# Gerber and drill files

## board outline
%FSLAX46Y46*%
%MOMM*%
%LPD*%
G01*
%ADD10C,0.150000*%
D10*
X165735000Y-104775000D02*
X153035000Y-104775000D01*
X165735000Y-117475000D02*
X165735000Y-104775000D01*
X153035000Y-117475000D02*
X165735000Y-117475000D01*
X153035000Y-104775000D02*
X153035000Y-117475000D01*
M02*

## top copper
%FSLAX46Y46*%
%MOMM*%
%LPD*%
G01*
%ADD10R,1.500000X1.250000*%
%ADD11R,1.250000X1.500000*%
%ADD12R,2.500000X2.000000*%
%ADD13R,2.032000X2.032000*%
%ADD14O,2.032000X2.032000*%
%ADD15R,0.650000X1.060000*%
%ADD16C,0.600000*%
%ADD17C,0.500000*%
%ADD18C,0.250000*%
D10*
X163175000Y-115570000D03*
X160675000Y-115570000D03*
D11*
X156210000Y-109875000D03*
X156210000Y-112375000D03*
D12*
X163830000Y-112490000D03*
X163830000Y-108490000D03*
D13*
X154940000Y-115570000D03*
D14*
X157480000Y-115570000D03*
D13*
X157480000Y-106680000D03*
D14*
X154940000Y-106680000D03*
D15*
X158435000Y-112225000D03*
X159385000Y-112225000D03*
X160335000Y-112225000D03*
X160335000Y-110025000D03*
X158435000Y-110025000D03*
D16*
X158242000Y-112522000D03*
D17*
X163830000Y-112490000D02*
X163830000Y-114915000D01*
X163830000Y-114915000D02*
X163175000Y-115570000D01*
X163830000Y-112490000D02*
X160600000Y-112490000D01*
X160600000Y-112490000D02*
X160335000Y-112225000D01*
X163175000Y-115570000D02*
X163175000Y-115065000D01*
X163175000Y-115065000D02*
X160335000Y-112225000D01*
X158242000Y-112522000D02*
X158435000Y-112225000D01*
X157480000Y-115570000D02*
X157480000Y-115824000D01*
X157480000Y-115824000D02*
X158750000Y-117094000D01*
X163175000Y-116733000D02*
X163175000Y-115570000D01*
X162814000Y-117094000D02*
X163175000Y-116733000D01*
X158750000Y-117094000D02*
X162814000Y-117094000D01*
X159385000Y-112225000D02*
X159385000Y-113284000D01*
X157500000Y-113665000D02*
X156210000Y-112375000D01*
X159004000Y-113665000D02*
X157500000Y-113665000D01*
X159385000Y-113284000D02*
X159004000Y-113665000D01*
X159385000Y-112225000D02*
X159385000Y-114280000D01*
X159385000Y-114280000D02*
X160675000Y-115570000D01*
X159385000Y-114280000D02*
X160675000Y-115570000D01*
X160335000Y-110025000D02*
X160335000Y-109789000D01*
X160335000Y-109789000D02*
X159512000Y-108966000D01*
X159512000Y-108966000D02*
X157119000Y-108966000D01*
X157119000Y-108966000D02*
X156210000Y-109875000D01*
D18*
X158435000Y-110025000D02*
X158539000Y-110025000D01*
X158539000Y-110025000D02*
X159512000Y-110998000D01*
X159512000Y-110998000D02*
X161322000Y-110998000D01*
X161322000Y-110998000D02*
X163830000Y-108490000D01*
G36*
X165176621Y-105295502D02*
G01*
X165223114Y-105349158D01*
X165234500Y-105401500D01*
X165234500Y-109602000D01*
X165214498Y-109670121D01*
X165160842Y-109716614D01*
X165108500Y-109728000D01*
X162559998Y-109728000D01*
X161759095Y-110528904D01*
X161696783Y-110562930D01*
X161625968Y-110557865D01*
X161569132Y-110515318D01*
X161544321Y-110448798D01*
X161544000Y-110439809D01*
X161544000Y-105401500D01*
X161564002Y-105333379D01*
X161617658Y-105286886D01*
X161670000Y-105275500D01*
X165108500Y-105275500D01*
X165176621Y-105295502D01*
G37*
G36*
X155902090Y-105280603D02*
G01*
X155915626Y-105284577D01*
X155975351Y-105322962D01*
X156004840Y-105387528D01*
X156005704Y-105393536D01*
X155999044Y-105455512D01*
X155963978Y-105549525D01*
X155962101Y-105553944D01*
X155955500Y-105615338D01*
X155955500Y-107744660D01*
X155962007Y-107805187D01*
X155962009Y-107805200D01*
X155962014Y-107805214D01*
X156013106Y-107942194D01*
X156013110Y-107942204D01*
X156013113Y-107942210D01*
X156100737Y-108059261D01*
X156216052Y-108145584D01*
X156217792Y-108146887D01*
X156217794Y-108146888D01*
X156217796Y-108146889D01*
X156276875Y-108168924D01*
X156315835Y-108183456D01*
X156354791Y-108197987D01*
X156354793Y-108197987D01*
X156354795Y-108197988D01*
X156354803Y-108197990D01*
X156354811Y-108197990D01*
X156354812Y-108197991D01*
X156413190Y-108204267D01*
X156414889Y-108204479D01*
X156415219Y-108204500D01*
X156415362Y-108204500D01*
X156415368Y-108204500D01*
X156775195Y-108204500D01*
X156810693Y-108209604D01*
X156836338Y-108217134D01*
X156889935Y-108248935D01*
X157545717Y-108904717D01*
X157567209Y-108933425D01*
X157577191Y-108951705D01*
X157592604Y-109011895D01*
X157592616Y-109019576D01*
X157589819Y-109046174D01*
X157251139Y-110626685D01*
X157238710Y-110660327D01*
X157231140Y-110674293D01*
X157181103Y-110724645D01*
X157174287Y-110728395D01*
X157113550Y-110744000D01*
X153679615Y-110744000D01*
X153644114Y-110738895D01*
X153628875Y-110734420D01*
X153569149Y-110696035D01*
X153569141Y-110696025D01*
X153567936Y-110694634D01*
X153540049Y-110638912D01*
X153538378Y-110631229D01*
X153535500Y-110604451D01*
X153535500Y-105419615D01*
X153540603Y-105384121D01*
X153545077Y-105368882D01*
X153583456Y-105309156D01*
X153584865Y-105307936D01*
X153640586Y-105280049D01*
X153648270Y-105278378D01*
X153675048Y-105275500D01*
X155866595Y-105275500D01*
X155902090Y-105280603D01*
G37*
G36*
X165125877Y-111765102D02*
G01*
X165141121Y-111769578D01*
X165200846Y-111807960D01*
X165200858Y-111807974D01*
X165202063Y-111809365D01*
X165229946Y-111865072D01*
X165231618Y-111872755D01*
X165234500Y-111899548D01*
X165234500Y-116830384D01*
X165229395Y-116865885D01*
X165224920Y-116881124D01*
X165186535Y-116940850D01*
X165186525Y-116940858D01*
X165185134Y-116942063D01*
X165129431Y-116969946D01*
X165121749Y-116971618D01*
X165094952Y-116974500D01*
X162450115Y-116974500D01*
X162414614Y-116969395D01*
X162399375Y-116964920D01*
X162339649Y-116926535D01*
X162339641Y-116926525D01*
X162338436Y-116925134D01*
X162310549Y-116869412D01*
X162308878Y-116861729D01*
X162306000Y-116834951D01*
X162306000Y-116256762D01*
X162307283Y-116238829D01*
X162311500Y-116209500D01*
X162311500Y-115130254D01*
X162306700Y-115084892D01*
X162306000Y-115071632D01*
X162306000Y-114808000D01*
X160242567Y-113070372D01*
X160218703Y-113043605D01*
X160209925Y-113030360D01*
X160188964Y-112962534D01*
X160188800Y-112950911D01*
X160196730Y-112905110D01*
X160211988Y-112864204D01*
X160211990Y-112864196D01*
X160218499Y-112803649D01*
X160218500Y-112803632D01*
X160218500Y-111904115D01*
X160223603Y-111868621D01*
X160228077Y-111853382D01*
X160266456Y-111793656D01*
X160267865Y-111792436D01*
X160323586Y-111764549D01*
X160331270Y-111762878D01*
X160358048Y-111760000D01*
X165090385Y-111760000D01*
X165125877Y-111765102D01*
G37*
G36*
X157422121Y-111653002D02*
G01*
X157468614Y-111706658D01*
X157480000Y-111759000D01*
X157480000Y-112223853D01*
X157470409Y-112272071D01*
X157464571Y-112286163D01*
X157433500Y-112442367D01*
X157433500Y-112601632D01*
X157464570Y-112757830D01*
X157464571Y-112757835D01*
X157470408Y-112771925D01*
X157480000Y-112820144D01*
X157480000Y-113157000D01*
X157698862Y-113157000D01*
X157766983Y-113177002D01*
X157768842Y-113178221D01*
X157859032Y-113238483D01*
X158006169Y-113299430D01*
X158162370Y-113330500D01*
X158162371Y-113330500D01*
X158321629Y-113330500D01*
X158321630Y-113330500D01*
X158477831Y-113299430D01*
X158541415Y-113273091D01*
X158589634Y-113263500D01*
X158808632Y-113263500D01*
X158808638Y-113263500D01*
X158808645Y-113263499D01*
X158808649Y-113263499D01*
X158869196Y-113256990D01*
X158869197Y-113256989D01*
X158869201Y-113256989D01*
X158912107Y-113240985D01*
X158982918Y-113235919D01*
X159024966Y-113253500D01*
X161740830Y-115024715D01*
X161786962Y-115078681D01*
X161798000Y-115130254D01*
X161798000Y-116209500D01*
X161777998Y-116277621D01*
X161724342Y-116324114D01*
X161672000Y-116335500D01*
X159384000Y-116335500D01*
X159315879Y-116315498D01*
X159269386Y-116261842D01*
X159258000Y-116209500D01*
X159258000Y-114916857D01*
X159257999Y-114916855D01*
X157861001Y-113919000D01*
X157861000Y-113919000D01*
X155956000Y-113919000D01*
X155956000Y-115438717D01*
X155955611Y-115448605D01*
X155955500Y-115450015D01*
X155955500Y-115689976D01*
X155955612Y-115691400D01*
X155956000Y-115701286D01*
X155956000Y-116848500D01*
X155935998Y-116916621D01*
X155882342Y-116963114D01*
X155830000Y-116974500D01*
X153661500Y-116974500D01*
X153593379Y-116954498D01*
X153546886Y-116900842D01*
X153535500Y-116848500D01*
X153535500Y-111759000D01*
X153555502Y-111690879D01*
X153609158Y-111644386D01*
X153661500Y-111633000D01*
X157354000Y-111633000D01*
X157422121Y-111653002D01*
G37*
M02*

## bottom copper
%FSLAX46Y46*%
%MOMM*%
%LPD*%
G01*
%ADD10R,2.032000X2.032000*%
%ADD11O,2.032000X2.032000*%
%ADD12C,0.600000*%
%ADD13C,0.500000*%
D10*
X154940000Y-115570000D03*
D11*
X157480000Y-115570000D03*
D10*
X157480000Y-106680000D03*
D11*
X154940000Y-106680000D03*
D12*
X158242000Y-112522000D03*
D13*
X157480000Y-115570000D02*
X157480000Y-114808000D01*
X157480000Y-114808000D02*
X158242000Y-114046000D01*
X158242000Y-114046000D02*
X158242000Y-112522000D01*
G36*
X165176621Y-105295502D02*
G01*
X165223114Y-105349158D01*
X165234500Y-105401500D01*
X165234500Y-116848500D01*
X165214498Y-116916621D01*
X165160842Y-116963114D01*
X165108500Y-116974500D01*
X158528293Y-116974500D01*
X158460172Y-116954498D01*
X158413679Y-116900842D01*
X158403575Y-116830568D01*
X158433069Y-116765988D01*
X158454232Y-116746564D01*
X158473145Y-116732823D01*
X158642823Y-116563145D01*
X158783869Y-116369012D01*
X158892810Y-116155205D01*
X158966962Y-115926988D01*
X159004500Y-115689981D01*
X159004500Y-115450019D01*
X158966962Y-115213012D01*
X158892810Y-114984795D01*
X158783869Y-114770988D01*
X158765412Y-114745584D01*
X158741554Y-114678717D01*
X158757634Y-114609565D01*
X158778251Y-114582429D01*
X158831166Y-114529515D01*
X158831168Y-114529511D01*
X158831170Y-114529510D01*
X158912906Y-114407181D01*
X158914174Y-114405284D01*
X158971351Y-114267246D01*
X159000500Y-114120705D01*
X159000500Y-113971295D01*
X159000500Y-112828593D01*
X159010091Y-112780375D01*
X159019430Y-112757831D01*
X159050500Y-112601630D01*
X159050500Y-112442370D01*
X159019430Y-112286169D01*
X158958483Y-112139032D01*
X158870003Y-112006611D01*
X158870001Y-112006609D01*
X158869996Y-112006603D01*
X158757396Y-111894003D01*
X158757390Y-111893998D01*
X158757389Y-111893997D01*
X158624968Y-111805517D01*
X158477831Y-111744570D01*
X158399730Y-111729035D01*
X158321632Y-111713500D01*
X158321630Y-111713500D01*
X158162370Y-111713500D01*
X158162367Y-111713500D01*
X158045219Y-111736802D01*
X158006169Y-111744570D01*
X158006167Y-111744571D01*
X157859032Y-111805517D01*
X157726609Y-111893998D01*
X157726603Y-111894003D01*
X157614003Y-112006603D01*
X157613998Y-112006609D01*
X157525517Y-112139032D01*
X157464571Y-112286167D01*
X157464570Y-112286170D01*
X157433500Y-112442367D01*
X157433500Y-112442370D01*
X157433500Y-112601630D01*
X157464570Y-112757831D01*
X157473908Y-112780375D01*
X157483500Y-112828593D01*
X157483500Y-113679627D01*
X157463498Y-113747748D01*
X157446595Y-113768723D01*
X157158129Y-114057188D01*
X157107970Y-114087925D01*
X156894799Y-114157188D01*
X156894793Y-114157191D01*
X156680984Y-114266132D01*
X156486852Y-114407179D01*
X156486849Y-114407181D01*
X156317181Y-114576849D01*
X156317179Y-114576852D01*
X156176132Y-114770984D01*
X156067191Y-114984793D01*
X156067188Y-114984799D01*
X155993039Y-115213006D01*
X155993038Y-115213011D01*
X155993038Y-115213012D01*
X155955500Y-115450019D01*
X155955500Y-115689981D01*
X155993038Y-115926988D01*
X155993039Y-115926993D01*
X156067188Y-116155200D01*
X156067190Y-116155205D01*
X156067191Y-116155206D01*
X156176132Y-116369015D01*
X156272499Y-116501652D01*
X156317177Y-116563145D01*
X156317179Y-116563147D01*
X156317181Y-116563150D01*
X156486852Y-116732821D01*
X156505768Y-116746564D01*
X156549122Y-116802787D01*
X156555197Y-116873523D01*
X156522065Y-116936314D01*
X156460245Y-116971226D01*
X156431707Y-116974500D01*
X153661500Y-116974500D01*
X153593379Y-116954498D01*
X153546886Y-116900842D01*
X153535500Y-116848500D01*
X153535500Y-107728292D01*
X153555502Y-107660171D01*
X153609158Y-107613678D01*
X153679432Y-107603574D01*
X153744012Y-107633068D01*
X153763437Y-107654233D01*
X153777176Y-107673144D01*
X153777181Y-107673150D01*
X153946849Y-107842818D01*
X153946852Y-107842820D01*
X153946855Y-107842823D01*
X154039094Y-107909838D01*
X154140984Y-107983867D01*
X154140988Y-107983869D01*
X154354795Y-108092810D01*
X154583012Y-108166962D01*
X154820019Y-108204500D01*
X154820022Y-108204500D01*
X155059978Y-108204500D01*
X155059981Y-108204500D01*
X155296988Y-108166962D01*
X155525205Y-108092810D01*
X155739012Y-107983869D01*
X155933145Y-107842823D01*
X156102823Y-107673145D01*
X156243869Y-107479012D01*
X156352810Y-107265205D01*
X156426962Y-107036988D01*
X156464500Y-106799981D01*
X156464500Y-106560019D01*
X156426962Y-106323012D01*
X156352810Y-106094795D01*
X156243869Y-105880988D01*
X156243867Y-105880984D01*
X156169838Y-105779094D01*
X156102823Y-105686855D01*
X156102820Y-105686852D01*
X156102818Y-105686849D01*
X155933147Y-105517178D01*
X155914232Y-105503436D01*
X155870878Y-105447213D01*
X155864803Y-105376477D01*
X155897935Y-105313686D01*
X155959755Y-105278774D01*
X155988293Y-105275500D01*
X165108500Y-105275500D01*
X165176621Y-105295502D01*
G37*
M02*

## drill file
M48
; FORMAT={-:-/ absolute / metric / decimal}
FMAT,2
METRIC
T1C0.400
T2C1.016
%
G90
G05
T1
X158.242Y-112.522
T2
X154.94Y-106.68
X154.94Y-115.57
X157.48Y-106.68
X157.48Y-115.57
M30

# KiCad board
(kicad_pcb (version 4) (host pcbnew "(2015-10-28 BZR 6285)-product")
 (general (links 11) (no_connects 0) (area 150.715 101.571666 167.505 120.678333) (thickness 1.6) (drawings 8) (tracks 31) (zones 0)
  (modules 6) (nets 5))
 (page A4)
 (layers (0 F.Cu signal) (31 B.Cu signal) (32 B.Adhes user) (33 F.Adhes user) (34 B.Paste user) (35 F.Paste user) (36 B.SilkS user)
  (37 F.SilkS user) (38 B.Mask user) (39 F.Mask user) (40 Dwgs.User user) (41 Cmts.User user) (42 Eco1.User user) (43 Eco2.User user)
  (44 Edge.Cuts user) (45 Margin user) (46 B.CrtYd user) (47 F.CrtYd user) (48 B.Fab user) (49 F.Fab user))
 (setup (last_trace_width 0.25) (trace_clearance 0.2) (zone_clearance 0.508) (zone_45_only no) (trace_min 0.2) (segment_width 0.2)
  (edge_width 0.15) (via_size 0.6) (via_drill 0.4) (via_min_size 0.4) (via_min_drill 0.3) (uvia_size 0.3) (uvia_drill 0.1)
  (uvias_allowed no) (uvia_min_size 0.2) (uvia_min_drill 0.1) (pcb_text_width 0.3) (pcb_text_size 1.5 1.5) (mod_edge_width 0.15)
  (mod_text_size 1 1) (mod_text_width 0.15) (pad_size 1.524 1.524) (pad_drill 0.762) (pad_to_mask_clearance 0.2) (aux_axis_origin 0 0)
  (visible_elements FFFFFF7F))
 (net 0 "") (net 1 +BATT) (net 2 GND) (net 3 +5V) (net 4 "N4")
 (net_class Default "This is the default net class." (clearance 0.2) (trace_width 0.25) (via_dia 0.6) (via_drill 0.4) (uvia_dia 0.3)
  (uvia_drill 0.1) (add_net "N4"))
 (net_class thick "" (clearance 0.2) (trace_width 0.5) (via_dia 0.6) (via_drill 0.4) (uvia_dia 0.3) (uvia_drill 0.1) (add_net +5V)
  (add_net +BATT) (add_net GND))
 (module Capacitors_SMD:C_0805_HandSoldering (layer F.Cu) (at 161.925 115.57 180) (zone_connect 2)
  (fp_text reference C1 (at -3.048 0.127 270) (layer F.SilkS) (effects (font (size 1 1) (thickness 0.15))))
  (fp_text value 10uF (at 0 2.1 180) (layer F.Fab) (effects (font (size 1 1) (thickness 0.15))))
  (pad 1 smd rect (at -1.25 0 180) (size 1.5 1.25) (layers F.Cu F.Paste F.Mask) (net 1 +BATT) (zone_connect 2))
  (pad 2 smd rect (at 1.25 0 180) (size 1.5 1.25) (layers F.Cu F.Paste F.Mask) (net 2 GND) (zone_connect 2)))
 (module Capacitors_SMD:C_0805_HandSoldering (layer F.Cu) (at 156.21 111.125 270) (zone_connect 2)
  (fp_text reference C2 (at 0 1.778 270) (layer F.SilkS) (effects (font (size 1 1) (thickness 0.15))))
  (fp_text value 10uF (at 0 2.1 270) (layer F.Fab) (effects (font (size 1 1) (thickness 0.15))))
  (pad 1 smd rect (at -1.25 0 270) (size 1.5 1.25) (layers F.Cu F.Paste F.Mask) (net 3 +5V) (zone_connect 2))
  (pad 2 smd rect (at 1.25 0 270) (size 1.5 1.25) (layers F.Cu F.Paste F.Mask) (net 2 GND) (zone_connect 2)))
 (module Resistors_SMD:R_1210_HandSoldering (layer F.Cu) (at 163.83 110.49 90) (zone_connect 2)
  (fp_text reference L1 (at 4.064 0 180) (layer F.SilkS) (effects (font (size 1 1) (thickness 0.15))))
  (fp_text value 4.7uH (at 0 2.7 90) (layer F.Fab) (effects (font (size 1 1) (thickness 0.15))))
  (pad 1 smd rect (at -2 0 90) (size 2 2.5) (layers F.Cu F.Paste F.Mask) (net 1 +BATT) (zone_connect 2))
  (pad 2 smd rect (at 2 0 90) (size 2 2.5) (layers F.Cu F.Paste F.Mask) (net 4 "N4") (zone_connect 2)))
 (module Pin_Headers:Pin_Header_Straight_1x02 (layer B.Cu) (at 154.94 115.57 270) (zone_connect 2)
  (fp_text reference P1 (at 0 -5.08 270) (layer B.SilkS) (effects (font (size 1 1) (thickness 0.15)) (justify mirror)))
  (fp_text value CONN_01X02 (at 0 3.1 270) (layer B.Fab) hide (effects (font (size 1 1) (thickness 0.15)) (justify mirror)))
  (pad 1 thru_hole rect (at 0 0 270) (size 2.032 2.032) (drill 1.016) (layers *.Cu *.Mask B.SilkS) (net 2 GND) (zone_connect 2))
  (pad 2 thru_hole oval (at 0 -2.54 270) (size 2.032 2.032) (drill 1.016) (layers *.Cu *.Mask B.SilkS) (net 1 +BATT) (zone_connect 2)))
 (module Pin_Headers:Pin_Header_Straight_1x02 (layer B.Cu) (at 157.48 106.68 90) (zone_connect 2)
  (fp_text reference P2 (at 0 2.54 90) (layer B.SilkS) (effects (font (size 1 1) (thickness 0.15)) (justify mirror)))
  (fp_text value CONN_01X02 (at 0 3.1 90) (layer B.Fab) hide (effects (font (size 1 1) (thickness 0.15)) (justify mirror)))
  (pad 1 thru_hole rect (at 0 0 90) (size 2.032 2.032) (drill 1.016) (layers *.Cu *.Mask B.SilkS) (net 2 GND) (zone_connect 2))
  (pad 2 thru_hole oval (at 0 -2.54 90) (size 2.032 2.032) (drill 1.016) (layers *.Cu *.Mask B.SilkS) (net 3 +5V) (zone_connect 2)))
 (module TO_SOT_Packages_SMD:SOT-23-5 (layer F.Cu) (at 159.385 111.125 90) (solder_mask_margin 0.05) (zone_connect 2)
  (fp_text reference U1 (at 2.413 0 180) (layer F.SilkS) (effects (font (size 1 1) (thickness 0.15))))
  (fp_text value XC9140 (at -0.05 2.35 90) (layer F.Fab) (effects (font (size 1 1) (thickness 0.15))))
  (pad 1 smd rect (at -1.1 -0.95 90) (size 1.06 0.65) (layers F.Cu F.Paste F.Mask) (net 1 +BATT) (zone_connect 2))
  (pad 2 smd rect (at -1.1 0 90) (size 1.06 0.65) (layers F.Cu F.Paste F.Mask) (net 2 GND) (zone_connect 2))
  (pad 3 smd rect (at -1.1 0.95 90) (size 1.06 0.65) (layers F.Cu F.Paste F.Mask) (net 1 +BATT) (zone_connect 2))
  (pad 4 smd rect (at 1.1 0.95 90) (size 1.06 0.65) (layers F.Cu F.Paste F.Mask) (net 3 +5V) (zone_connect 2))
  (pad 5 smd rect (at 1.1 -0.95 90) (size 1.06 0.65) (layers F.Cu F.Paste F.Mask) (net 4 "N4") (zone_connect 2)))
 (gr_line (start 165.735 104.775) (end 153.035 104.775) (angle 90) (layer Edge.Cuts) (width 0.15))
 (gr_line (start 165.735 117.475) (end 165.735 104.775) (angle 90) (layer Edge.Cuts) (width 0.15))
 (gr_line (start 153.035 117.475) (end 165.735 117.475) (angle 90) (layer Edge.Cuts) (width 0.15))
 (gr_line (start 153.035 104.775) (end 153.035 117.475) (angle 90) (layer Edge.Cuts) (width 0.15))
 (segment (start 163.83 112.49) (end 163.83 114.915) (width 0.5) (layer F.Cu) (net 1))
 (segment (start 163.83 114.915) (end 163.175 115.57) (width 0.5) (layer F.Cu) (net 1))
 (segment (start 163.83 112.49) (end 160.6 112.49) (width 0.5) (layer F.Cu) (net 1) (status 20))
 (segment (start 160.6 112.49) (end 160.335 112.225) (width 0.5) (layer F.Cu) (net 1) (status 30))
 (segment (start 163.175 115.57) (end 163.175 115.065) (width 0.5) (layer F.Cu) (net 1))
 (segment (start 163.175 115.065) (end 160.335 112.225) (width 0.5) (layer F.Cu) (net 1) (status 20))
 (segment (start 157.48 115.57) (end 157.48 114.808) (width 0.5) (layer B.Cu) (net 1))
 (segment (start 157.48 114.808) (end 158.242 114.046) (width 0.5) (layer B.Cu) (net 1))
 (segment (start 158.242 112.522) (end 158.435 112.225) (width 0.5) (layer F.Cu) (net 1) (status 30))
 (via (at 158.242 112.522) (size 0.6) (drill 0.4) (layers F.Cu B.Cu) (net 1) (status 30))
 (segment (start 158.242 114.046) (end 158.242 112.522) (width 0.5) (layer B.Cu) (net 1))
 (segment (start 157.48 115.57) (end 157.48 115.824) (width 0.5) (layer F.Cu) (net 1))
 (segment (start 157.48 115.824) (end 158.75 117.094) (width 0.5) (layer F.Cu) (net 1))
 (segment (start 163.175 116.733) (end 163.175 115.57) (width 0.5) (layer F.Cu) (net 1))
 (segment (start 162.814 117.094) (end 163.175 116.733) (width 0.5) (layer F.Cu) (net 1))
 (segment (start 158.75 117.094) (end 162.814 117.094) (width 0.5) (layer F.Cu) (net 1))
 (segment (start 159.385 112.225) (end 159.385 113.284) (width 0.5) (layer F.Cu) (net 2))
 (segment (start 157.5 113.665) (end 156.21 112.375) (width 0.5) (layer F.Cu) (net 2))
 (segment (start 159.004 113.665) (end 157.5 113.665) (width 0.5) (layer F.Cu) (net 2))
 (segment (start 159.385 113.284) (end 159.004 113.665) (width 0.5) (layer F.Cu) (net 2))
 (segment (start 159.385 112.225) (end 159.385 114.28) (width 0.5) (layer F.Cu) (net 2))
 (segment (start 159.385 114.28) (end 160.675 115.57) (width 0.5) (layer F.Cu) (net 2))
 (segment (start 159.385 114.28) (end 160.675 115.57) (width 0.5) (layer F.Cu) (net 2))
 (segment (start 160.335 110.025) (end 160.335 109.789) (width 0.5) (layer F.Cu) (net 3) (status 30))
 (segment (start 160.335 109.789) (end 159.512 108.966) (width 0.5) (layer F.Cu) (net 3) (status 10))
 (segment (start 159.512 108.966) (end 157.119 108.966) (width 0.5) (layer F.Cu) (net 3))
 (segment (start 157.119 108.966) (end 156.21 109.875) (width 0.5) (layer F.Cu) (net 3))
 (segment (start 158.435 110.025) (end 158.539 110.025) (width 0.25) (layer F.Cu) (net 4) (status 30))
 (segment (start 158.539 110.025) (end 159.512 110.998) (width 0.25) (layer F.Cu) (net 4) (status 10))
 (segment (start 159.512 110.998) (end 161.322 110.998) (width 0.25) (layer F.Cu) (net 4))
 (segment (start 161.322 110.998) (end 163.83 108.49) (width 0.25) (layer F.Cu) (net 4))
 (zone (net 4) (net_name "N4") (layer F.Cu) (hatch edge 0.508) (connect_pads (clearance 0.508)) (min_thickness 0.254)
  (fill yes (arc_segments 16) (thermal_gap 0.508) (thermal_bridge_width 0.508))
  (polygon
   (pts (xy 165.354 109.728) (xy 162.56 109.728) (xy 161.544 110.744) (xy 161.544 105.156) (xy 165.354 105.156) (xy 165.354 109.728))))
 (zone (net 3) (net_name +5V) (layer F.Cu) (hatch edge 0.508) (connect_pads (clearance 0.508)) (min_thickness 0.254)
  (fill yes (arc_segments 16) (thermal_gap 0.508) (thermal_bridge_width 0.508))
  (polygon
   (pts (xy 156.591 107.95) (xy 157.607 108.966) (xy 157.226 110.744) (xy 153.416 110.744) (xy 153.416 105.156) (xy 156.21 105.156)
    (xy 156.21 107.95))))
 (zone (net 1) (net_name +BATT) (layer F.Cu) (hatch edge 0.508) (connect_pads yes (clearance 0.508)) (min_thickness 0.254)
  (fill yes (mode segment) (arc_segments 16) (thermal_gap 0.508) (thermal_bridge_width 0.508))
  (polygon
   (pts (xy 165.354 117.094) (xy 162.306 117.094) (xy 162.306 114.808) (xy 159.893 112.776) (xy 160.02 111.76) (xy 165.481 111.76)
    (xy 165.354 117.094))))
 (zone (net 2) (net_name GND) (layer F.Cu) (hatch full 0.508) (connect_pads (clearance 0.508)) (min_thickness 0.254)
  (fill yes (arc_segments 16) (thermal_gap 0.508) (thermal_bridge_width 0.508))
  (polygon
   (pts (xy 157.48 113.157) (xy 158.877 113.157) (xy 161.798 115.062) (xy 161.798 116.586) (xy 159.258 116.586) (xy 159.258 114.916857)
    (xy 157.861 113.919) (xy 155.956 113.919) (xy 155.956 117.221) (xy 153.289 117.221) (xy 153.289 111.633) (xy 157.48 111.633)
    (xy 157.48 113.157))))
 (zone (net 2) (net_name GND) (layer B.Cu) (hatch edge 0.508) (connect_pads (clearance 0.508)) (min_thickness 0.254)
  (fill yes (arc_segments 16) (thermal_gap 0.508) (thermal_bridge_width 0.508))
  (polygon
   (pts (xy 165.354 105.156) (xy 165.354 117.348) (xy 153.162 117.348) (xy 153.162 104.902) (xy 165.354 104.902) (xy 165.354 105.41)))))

